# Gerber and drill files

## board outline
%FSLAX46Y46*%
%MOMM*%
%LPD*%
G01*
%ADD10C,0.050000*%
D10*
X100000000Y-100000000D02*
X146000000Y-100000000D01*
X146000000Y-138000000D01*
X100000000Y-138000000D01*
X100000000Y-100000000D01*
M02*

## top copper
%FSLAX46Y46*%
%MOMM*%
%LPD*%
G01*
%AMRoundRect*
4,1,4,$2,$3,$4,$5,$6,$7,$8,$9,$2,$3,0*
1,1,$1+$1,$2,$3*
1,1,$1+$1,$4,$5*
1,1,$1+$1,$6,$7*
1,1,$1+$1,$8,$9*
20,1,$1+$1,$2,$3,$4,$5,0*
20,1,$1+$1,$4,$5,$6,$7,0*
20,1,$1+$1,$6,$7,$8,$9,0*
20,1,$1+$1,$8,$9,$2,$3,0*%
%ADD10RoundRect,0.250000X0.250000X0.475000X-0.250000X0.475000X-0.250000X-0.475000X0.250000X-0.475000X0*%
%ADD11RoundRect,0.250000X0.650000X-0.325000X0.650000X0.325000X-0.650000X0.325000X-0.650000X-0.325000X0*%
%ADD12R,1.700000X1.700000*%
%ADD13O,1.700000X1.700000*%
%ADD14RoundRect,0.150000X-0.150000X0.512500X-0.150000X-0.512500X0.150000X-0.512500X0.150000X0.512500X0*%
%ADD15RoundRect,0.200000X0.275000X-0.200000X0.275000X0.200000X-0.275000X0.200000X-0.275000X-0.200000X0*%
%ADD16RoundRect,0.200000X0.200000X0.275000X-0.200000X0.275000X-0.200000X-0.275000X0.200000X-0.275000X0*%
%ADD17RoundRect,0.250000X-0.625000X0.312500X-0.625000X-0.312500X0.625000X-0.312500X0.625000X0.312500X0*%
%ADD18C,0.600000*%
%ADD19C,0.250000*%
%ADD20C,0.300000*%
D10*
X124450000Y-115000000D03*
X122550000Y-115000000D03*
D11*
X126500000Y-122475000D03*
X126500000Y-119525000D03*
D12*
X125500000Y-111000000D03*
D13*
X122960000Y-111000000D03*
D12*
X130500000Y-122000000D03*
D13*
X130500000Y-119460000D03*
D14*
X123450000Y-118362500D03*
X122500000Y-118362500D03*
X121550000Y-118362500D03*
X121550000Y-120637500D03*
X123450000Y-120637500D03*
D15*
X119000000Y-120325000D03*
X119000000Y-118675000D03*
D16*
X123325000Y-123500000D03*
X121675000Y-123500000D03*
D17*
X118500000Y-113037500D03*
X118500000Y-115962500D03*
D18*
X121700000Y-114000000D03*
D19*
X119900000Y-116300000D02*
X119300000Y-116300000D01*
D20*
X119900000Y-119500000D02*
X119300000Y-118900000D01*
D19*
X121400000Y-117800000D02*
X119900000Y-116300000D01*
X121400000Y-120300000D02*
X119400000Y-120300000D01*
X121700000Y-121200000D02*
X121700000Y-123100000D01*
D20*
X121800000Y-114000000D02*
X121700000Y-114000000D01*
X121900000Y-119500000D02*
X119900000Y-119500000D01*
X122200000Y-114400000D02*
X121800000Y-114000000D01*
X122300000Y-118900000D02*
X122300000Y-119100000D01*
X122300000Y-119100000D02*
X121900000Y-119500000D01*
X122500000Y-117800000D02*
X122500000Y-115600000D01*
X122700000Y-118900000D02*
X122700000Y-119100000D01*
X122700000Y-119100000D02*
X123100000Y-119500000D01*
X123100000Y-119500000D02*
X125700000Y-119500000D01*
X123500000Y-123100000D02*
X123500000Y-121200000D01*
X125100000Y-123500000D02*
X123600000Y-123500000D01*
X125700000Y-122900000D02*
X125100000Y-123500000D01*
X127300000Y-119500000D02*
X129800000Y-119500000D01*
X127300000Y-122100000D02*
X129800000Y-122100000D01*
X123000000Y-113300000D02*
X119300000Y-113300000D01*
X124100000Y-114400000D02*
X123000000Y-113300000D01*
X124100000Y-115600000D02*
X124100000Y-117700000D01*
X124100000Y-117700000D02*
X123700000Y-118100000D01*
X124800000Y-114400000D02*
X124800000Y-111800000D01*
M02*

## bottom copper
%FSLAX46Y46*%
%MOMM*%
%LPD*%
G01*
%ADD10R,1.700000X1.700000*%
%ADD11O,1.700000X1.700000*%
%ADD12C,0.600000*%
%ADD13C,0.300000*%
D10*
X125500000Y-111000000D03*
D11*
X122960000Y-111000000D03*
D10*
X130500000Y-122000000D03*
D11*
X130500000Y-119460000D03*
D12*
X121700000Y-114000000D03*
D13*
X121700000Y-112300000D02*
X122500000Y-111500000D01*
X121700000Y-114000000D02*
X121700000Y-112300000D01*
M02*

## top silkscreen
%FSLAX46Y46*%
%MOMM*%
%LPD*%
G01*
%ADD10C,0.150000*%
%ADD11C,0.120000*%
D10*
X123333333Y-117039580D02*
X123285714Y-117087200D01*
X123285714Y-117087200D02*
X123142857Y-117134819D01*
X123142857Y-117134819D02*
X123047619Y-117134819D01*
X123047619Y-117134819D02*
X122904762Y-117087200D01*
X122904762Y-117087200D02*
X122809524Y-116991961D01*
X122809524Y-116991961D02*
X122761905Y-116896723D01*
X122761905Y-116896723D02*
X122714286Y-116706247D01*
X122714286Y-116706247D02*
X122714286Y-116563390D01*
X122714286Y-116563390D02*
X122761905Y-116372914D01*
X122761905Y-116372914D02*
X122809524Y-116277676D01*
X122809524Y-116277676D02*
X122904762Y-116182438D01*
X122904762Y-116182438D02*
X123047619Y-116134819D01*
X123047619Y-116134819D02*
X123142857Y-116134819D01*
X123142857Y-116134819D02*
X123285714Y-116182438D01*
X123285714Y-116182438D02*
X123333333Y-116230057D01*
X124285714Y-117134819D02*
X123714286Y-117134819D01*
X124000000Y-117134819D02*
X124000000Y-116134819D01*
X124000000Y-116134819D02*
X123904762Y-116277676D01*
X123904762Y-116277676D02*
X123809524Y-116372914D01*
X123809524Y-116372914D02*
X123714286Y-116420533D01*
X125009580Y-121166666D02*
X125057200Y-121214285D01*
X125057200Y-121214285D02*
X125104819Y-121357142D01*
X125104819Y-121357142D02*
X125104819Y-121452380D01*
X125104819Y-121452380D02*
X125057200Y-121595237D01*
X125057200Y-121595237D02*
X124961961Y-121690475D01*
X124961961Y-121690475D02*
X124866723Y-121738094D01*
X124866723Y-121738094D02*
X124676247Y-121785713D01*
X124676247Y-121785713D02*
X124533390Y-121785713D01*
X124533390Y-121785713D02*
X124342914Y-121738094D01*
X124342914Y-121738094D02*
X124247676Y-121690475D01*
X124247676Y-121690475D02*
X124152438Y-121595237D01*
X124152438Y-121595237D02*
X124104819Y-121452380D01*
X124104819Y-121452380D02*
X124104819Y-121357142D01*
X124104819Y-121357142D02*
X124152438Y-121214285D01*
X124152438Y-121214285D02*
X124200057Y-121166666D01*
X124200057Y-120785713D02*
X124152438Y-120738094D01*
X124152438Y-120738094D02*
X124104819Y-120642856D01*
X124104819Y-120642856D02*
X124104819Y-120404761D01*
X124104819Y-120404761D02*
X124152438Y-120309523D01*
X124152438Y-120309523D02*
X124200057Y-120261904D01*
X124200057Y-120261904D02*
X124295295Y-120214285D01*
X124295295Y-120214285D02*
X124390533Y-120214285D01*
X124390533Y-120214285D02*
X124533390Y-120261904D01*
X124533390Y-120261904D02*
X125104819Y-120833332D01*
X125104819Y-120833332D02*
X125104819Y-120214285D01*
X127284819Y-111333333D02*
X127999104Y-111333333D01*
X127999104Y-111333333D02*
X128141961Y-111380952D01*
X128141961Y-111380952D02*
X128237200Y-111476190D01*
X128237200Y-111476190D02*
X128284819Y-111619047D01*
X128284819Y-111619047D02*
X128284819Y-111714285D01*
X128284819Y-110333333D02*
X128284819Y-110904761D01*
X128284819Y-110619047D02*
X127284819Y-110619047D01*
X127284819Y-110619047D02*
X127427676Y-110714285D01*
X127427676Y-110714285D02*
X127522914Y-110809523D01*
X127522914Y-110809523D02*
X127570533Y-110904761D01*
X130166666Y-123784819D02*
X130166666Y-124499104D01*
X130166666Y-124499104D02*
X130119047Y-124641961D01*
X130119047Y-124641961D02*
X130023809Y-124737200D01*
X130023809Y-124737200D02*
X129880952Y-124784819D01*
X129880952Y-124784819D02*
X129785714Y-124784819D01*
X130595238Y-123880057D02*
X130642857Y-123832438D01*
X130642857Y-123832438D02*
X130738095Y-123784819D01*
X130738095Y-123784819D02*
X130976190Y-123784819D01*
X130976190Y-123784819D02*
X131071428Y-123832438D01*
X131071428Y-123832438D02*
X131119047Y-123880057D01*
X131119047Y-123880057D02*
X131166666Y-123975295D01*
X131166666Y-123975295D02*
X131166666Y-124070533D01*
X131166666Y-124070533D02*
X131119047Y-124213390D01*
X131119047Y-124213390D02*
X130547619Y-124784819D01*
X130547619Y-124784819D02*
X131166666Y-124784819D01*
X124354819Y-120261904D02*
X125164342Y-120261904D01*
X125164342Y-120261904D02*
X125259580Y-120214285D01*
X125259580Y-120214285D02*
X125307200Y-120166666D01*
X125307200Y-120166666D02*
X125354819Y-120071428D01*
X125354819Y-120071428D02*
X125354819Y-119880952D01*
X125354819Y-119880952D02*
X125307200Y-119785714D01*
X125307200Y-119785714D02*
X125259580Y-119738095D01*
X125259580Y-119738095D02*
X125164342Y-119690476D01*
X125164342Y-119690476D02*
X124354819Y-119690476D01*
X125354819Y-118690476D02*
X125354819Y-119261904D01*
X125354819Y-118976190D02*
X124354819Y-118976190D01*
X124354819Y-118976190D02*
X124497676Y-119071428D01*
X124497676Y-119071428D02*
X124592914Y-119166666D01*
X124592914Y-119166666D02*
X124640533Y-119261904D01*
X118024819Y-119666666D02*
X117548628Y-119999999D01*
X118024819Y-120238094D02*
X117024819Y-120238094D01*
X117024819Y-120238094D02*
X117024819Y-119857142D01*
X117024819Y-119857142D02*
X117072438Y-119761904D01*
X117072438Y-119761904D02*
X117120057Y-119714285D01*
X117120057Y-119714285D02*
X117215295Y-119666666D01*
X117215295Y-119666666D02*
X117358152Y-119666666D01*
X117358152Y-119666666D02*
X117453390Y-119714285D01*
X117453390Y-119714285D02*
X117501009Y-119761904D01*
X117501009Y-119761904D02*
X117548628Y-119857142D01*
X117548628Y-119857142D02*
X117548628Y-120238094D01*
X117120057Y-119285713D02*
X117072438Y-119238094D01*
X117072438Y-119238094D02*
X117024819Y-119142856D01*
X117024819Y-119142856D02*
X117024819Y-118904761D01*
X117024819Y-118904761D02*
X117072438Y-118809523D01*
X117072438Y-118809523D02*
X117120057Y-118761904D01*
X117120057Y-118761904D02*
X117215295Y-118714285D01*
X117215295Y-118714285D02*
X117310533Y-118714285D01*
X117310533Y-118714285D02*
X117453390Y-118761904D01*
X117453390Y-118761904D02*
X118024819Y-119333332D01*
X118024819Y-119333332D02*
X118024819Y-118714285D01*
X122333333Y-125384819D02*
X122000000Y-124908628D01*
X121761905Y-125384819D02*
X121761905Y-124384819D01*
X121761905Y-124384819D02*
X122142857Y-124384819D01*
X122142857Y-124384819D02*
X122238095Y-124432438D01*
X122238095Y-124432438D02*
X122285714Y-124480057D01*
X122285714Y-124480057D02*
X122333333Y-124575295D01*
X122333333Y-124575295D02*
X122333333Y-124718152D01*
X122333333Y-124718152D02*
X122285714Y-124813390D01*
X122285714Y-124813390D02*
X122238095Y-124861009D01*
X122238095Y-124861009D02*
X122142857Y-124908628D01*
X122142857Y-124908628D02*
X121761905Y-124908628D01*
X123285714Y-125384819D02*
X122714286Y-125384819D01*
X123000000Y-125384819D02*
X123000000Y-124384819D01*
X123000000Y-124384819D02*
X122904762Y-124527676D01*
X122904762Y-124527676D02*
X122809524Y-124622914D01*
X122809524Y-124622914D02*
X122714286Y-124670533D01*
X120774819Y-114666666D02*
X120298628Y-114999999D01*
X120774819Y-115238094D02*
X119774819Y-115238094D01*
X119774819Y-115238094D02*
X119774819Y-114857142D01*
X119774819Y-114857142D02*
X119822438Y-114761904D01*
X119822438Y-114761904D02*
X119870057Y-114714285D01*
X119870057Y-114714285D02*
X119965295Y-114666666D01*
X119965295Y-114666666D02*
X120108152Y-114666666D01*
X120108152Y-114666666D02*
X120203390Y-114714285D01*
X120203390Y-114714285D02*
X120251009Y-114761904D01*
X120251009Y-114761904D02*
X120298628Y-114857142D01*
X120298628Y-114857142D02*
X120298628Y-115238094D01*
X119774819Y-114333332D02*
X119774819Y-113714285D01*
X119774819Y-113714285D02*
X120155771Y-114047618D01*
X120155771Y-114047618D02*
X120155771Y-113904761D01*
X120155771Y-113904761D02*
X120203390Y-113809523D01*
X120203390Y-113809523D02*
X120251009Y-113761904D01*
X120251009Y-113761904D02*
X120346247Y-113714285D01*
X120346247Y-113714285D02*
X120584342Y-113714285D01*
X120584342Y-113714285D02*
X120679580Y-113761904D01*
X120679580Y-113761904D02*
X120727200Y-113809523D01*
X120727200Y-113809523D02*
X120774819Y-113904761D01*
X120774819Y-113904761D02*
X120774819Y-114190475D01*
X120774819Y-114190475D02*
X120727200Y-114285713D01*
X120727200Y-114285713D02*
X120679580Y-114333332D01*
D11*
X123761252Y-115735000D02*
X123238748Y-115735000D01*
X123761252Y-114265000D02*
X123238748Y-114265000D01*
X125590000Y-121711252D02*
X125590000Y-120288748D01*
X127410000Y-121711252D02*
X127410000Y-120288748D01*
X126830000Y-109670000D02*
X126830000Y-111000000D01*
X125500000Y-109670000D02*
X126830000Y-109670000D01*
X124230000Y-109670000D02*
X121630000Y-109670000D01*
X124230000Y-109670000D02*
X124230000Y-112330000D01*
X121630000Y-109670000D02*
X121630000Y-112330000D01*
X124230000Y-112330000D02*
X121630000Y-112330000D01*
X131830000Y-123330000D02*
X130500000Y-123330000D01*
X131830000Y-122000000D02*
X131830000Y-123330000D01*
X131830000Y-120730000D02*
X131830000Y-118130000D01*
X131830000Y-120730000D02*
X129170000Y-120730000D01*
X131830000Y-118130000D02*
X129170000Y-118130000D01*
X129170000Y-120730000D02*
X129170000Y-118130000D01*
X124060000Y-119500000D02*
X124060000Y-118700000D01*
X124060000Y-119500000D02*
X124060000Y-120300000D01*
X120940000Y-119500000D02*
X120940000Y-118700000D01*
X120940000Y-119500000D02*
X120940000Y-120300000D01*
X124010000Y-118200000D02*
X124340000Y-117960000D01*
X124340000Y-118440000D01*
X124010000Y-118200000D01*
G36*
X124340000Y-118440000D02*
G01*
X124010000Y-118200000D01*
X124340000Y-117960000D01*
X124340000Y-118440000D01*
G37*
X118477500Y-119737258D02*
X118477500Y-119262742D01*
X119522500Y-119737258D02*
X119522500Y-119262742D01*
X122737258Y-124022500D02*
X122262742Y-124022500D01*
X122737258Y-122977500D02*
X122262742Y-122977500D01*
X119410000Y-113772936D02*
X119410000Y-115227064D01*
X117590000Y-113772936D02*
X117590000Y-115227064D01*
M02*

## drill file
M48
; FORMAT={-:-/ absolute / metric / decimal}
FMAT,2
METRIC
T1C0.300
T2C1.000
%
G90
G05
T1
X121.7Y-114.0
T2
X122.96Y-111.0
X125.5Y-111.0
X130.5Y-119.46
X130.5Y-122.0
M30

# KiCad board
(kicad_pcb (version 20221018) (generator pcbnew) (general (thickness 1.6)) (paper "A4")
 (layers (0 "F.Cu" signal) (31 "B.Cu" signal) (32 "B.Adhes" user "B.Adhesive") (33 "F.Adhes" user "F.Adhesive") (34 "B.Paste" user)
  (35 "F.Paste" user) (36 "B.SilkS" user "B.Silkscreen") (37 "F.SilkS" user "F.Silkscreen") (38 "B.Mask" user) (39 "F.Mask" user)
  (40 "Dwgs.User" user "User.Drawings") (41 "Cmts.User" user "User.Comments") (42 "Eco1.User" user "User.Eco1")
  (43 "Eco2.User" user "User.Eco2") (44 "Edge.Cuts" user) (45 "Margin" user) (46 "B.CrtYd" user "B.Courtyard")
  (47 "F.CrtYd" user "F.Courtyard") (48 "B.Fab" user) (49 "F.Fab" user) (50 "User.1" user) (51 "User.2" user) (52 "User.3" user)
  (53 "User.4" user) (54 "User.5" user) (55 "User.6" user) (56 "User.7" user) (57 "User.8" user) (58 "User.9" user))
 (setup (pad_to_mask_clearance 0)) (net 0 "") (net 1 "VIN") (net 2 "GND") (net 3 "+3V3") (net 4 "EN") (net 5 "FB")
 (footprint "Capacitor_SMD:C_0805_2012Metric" (layer "F.Cu") (at 123.5 115 180)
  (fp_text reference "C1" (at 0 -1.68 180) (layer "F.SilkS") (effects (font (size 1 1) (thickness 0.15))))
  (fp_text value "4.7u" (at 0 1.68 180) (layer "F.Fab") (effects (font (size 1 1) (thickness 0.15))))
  (fp_line (start -0.261252 -0.735) (end 0.261252 -0.735) (stroke (width 0.12) (type solid)) (layer "F.SilkS"))
  (fp_line (start -0.261252 0.735) (end 0.261252 0.735) (stroke (width 0.12) (type solid)) (layer "F.SilkS"))
  (pad "1" smd roundrect (at -0.95 0 180) (size 1 1.45) (layers "F.Cu" "F.Paste" "F.Mask") (roundrect_rratio 0.25) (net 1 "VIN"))
  (pad "2" smd roundrect (at 0.95 0 180) (size 1 1.45) (layers "F.Cu" "F.Paste" "F.Mask") (roundrect_rratio 0.25) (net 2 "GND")))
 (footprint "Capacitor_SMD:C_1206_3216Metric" (layer "F.Cu") (at 126.5 121 90)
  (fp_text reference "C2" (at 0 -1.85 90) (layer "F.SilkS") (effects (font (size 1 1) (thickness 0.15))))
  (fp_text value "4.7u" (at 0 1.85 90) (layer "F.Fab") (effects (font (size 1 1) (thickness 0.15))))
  (fp_line (start -0.711252 -0.91) (end 0.711252 -0.91) (stroke (width 0.12) (type solid)) (layer "F.SilkS"))
  (fp_line (start -0.711252 0.91) (end 0.711252 0.91) (stroke (width 0.12) (type solid)) (layer "F.SilkS"))
  (pad "1" smd roundrect (at -1.475 0 90) (size 1.15 1.8) (layers "F.Cu" "F.Paste" "F.Mask") (roundrect_rratio 0.217391) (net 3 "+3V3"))
  (pad "2" smd roundrect (at 1.475 0 90) (size 1.15 1.8) (layers "F.Cu" "F.Paste" "F.Mask") (roundrect_rratio 0.217391) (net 2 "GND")))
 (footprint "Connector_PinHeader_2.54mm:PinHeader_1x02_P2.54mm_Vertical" (layer "F.Cu") (at 125.5 111 -90)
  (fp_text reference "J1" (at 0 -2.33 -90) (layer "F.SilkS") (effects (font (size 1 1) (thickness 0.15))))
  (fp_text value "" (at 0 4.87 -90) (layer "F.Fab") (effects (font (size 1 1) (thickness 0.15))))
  (fp_line (start -1.33 -1.33) (end 0 -1.33) (stroke (width 0.12) (type solid)) (layer "F.SilkS"))
  (fp_line (start -1.33 0) (end -1.33 -1.33) (stroke (width 0.12) (type solid)) (layer "F.SilkS"))
  (fp_line (start -1.33 1.27) (end -1.33 3.87) (stroke (width 0.12) (type solid)) (layer "F.SilkS"))
  (fp_line (start -1.33 1.27) (end 1.33 1.27) (stroke (width 0.12) (type solid)) (layer "F.SilkS"))
  (fp_line (start -1.33 3.87) (end 1.33 3.87) (stroke (width 0.12) (type solid)) (layer "F.SilkS"))
  (fp_line (start 1.33 1.27) (end 1.33 3.87) (stroke (width 0.12) (type solid)) (layer "F.SilkS"))
  (pad "1" thru_hole rect (at 0 0 270) (size 1.7 1.7) (drill 1) (layers "*.Cu" "*.Mask") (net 1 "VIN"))
  (pad "2" thru_hole oval (at 0 2.54 270) (size 1.7 1.7) (drill 1) (layers "*.Cu" "*.Mask") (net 2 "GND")))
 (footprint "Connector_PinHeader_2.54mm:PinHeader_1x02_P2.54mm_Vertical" (layer "F.Cu") (at 130.5 122 180)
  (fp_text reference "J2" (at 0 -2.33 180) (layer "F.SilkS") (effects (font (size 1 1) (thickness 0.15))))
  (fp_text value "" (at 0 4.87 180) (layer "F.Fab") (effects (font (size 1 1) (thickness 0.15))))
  (fp_line (start -1.33 -1.33) (end 0 -1.33) (stroke (width 0.12) (type solid)) (layer "F.SilkS"))
  (fp_line (start -1.33 0) (end -1.33 -1.33) (stroke (width 0.12) (type solid)) (layer "F.SilkS"))
  (fp_line (start -1.33 1.27) (end -1.33 3.87) (stroke (width 0.12) (type solid)) (layer "F.SilkS"))
  (fp_line (start -1.33 1.27) (end 1.33 1.27) (stroke (width 0.12) (type solid)) (layer "F.SilkS"))
  (fp_line (start -1.33 3.87) (end 1.33 3.87) (stroke (width 0.12) (type solid)) (layer "F.SilkS"))
  (fp_line (start 1.33 1.27) (end 1.33 3.87) (stroke (width 0.12) (type solid)) (layer "F.SilkS"))
  (pad "1" thru_hole rect (at 0 0 180) (size 1.7 1.7) (drill 1) (layers "*.Cu" "*.Mask") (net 3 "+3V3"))
  (pad "2" thru_hole oval (at 0 2.54 180) (size 1.7 1.7) (drill 1) (layers "*.Cu" "*.Mask") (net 2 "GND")))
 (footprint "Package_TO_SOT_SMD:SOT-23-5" (layer "F.Cu") (at 122.5 119.5 -90)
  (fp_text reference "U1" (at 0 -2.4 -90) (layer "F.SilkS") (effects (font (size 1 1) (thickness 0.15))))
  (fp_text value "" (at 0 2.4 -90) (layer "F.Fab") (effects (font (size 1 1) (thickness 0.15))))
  (fp_line (start 0 -1.56) (end -0.8 -1.56) (stroke (width 0.12) (type solid)) (layer "F.SilkS"))
  (fp_line (start 0 -1.56) (end 0.8 -1.56) (stroke (width 0.12) (type solid)) (layer "F.SilkS"))
  (fp_line (start 0 1.56) (end -0.8 1.56) (stroke (width 0.12) (type solid)) (layer "F.SilkS"))
  (fp_line (start 0 1.56) (end 0.8 1.56) (stroke (width 0.12) (type solid)) (layer "F.SilkS"))
  (fp_poly
   (pts (xy -1.3 -1.51) (xy -1.54 -1.84) (xy -1.06 -1.84) (xy -1.3 -1.51)) (stroke (width 0.12) (type solid)) (fill solid) (layer "F.SilkS"))
  (pad "1" smd roundrect (at -1.1375 -0.95 270) (size 1.325 0.6) (layers "F.Cu" "F.Paste" "F.Mask") (roundrect_rratio 0.25) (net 1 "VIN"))
  (pad "2" smd roundrect (at -1.1375 0 270) (size 1.325 0.6) (layers "F.Cu" "F.Paste" "F.Mask") (roundrect_rratio 0.25) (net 2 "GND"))
  (pad "3" smd roundrect (at -1.1375 0.95 270) (size 1.325 0.6) (layers "F.Cu" "F.Paste" "F.Mask") (roundrect_rratio 0.25) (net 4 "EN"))
  (pad "4" smd roundrect (at 1.1375 0.95 270) (size 1.325 0.6) (layers "F.Cu" "F.Paste" "F.Mask") (roundrect_rratio 0.25) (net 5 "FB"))
  (pad "5" smd roundrect (at 1.1375 -0.95 270) (size 1.325 0.6) (layers "F.Cu" "F.Paste" "F.Mask") (roundrect_rratio 0.25) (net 3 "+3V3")))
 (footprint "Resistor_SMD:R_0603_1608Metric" (layer "F.Cu") (at 119 119.5 90)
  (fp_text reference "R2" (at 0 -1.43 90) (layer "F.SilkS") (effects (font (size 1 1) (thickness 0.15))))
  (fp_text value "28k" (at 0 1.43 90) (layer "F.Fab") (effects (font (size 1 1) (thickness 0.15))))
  (fp_line (start -0.237258 -0.5225) (end 0.237258 -0.5225) (stroke (width 0.12) (type solid)) (layer "F.SilkS"))
  (fp_line (start -0.237258 0.5225) (end 0.237258 0.5225) (stroke (width 0.12) (type solid)) (layer "F.SilkS"))
  (pad "1" smd roundrect (at -0.825 0 90) (size 0.8 0.95) (layers "F.Cu" "F.Paste" "F.Mask") (roundrect_rratio 0.25) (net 5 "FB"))
  (pad "2" smd roundrect (at 0.825 0 90) (size 0.8 0.95) (layers "F.Cu" "F.Paste" "F.Mask") (roundrect_rratio 0.25) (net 2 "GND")))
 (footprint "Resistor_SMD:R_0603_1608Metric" (layer "F.Cu") (at 122.5 123.5 180)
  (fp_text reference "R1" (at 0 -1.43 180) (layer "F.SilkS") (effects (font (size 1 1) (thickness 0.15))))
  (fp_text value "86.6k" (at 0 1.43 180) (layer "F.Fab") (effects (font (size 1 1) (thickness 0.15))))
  (fp_line (start -0.237258 -0.5225) (end 0.237258 -0.5225) (stroke (width 0.12) (type solid)) (layer "F.SilkS"))
  (fp_line (start -0.237258 0.5225) (end 0.237258 0.5225) (stroke (width 0.12) (type solid)) (layer "F.SilkS"))
  (pad "1" smd roundrect (at -0.825 0 180) (size 0.8 0.95) (layers "F.Cu" "F.Paste" "F.Mask") (roundrect_rratio 0.25) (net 3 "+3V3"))
  (pad "2" smd roundrect (at 0.825 0 180) (size 0.8 0.95) (layers "F.Cu" "F.Paste" "F.Mask") (roundrect_rratio 0.25) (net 5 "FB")))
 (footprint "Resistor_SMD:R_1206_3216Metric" (layer "F.Cu") (at 118.5 114.5 -90)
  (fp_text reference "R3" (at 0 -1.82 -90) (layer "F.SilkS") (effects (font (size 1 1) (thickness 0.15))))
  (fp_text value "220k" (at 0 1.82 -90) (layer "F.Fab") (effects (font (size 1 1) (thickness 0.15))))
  (fp_line (start -0.727064 -0.91) (end 0.727064 -0.91) (stroke (width 0.12) (type solid)) (layer "F.SilkS"))
  (fp_line (start -0.727064 0.91) (end 0.727064 0.91) (stroke (width 0.12) (type solid)) (layer "F.SilkS"))
  (pad "1" smd roundrect (at -1.4625 0 270) (size 1.125 1.75) (layers "F.Cu" "F.Paste" "F.Mask") (roundrect_rratio 0.222222) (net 1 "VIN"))
  (pad "2" smd roundrect (at 1.4625 0 270) (size 1.125 1.75) (layers "F.Cu" "F.Paste" "F.Mask") (roundrect_rratio 0.222222) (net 4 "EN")))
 (gr_rect (start 100 100) (end 146 138) (stroke (width 0.05) (type default)) (fill none) (layer "Edge.Cuts"))
 (segment (start 119.9 116.3) (end 119.3 116.3) (width 0.25) (layer "F.Cu") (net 4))
 (segment (start 119.9 119.5) (end 119.3 118.9) (width 0.3) (layer "F.Cu") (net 2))
 (segment (start 121.4 117.8) (end 119.9 116.3) (width 0.25) (layer "F.Cu") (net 4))
 (segment (start 121.4 120.3) (end 119.4 120.3) (width 0.25) (layer "F.Cu") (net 5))
 (segment (start 121.7 121.2) (end 121.7 123.1) (width 0.25) (layer "F.Cu") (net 5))
 (segment (start 121.8 114) (end 121.7 114) (width 0.3) (layer "F.Cu") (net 2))
 (segment (start 121.9 119.5) (end 119.9 119.5) (width 0.3) (layer "F.Cu") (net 2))
 (segment (start 122.2 114.4) (end 121.8 114) (width 0.3) (layer "F.Cu") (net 2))
 (segment (start 122.3 118.9) (end 122.3 119.1) (width 0.3) (layer "F.Cu") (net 2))
 (segment (start 122.3 119.1) (end 121.9 119.5) (width 0.3) (layer "F.Cu") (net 2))
 (segment (start 122.5 117.8) (end 122.5 115.6) (width 0.3) (layer "F.Cu") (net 2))
 (segment (start 122.7 118.9) (end 122.7 119.1) (width 0.3) (layer "F.Cu") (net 2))
 (segment (start 122.7 119.1) (end 123.1 119.5) (width 0.3) (layer "F.Cu") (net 2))
 (segment (start 123.1 119.5) (end 125.7 119.5) (width 0.3) (layer "F.Cu") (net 2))
 (segment (start 123.5 123.1) (end 123.5 121.2) (width 0.3) (layer "F.Cu") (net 3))
 (segment (start 125.1 123.5) (end 123.6 123.5) (width 0.3) (layer "F.Cu") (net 3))
 (segment (start 125.7 122.9) (end 125.1 123.5) (width 0.3) (layer "F.Cu") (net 3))
 (segment (start 127.3 119.5) (end 129.8 119.5) (width 0.3) (layer "F.Cu") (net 2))
 (segment (start 127.3 122.1) (end 129.8 122.1) (width 0.3) (layer "F.Cu") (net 3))
 (via (at 121.7 114) (size 0.6) (drill 0.3) (layers "F.Cu" "B.Cu") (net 2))
 (segment (start 121.7 112.3) (end 122.5 111.5) (width 0.3) (layer "B.Cu") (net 2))
 (segment (start 121.7 114) (end 121.7 112.3) (width 0.3) (layer "B.Cu") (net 2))
 (segment (start 123 113.3) (end 119.3 113.3) (width 0.3) (layer "F.Cu") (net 1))
 (segment (start 124.1 114.4) (end 123 113.3) (width 0.3) (layer "F.Cu") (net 1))
 (segment (start 124.1 115.6) (end 124.1 117.7) (width 0.3) (layer "F.Cu") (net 1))
 (segment (start 124.1 117.7) (end 123.7 118.1) (width 0.3) (layer "F.Cu") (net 1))
 (segment (start 124.8 114.4) (end 124.8 111.8) (width 0.3) (layer "F.Cu") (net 1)))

